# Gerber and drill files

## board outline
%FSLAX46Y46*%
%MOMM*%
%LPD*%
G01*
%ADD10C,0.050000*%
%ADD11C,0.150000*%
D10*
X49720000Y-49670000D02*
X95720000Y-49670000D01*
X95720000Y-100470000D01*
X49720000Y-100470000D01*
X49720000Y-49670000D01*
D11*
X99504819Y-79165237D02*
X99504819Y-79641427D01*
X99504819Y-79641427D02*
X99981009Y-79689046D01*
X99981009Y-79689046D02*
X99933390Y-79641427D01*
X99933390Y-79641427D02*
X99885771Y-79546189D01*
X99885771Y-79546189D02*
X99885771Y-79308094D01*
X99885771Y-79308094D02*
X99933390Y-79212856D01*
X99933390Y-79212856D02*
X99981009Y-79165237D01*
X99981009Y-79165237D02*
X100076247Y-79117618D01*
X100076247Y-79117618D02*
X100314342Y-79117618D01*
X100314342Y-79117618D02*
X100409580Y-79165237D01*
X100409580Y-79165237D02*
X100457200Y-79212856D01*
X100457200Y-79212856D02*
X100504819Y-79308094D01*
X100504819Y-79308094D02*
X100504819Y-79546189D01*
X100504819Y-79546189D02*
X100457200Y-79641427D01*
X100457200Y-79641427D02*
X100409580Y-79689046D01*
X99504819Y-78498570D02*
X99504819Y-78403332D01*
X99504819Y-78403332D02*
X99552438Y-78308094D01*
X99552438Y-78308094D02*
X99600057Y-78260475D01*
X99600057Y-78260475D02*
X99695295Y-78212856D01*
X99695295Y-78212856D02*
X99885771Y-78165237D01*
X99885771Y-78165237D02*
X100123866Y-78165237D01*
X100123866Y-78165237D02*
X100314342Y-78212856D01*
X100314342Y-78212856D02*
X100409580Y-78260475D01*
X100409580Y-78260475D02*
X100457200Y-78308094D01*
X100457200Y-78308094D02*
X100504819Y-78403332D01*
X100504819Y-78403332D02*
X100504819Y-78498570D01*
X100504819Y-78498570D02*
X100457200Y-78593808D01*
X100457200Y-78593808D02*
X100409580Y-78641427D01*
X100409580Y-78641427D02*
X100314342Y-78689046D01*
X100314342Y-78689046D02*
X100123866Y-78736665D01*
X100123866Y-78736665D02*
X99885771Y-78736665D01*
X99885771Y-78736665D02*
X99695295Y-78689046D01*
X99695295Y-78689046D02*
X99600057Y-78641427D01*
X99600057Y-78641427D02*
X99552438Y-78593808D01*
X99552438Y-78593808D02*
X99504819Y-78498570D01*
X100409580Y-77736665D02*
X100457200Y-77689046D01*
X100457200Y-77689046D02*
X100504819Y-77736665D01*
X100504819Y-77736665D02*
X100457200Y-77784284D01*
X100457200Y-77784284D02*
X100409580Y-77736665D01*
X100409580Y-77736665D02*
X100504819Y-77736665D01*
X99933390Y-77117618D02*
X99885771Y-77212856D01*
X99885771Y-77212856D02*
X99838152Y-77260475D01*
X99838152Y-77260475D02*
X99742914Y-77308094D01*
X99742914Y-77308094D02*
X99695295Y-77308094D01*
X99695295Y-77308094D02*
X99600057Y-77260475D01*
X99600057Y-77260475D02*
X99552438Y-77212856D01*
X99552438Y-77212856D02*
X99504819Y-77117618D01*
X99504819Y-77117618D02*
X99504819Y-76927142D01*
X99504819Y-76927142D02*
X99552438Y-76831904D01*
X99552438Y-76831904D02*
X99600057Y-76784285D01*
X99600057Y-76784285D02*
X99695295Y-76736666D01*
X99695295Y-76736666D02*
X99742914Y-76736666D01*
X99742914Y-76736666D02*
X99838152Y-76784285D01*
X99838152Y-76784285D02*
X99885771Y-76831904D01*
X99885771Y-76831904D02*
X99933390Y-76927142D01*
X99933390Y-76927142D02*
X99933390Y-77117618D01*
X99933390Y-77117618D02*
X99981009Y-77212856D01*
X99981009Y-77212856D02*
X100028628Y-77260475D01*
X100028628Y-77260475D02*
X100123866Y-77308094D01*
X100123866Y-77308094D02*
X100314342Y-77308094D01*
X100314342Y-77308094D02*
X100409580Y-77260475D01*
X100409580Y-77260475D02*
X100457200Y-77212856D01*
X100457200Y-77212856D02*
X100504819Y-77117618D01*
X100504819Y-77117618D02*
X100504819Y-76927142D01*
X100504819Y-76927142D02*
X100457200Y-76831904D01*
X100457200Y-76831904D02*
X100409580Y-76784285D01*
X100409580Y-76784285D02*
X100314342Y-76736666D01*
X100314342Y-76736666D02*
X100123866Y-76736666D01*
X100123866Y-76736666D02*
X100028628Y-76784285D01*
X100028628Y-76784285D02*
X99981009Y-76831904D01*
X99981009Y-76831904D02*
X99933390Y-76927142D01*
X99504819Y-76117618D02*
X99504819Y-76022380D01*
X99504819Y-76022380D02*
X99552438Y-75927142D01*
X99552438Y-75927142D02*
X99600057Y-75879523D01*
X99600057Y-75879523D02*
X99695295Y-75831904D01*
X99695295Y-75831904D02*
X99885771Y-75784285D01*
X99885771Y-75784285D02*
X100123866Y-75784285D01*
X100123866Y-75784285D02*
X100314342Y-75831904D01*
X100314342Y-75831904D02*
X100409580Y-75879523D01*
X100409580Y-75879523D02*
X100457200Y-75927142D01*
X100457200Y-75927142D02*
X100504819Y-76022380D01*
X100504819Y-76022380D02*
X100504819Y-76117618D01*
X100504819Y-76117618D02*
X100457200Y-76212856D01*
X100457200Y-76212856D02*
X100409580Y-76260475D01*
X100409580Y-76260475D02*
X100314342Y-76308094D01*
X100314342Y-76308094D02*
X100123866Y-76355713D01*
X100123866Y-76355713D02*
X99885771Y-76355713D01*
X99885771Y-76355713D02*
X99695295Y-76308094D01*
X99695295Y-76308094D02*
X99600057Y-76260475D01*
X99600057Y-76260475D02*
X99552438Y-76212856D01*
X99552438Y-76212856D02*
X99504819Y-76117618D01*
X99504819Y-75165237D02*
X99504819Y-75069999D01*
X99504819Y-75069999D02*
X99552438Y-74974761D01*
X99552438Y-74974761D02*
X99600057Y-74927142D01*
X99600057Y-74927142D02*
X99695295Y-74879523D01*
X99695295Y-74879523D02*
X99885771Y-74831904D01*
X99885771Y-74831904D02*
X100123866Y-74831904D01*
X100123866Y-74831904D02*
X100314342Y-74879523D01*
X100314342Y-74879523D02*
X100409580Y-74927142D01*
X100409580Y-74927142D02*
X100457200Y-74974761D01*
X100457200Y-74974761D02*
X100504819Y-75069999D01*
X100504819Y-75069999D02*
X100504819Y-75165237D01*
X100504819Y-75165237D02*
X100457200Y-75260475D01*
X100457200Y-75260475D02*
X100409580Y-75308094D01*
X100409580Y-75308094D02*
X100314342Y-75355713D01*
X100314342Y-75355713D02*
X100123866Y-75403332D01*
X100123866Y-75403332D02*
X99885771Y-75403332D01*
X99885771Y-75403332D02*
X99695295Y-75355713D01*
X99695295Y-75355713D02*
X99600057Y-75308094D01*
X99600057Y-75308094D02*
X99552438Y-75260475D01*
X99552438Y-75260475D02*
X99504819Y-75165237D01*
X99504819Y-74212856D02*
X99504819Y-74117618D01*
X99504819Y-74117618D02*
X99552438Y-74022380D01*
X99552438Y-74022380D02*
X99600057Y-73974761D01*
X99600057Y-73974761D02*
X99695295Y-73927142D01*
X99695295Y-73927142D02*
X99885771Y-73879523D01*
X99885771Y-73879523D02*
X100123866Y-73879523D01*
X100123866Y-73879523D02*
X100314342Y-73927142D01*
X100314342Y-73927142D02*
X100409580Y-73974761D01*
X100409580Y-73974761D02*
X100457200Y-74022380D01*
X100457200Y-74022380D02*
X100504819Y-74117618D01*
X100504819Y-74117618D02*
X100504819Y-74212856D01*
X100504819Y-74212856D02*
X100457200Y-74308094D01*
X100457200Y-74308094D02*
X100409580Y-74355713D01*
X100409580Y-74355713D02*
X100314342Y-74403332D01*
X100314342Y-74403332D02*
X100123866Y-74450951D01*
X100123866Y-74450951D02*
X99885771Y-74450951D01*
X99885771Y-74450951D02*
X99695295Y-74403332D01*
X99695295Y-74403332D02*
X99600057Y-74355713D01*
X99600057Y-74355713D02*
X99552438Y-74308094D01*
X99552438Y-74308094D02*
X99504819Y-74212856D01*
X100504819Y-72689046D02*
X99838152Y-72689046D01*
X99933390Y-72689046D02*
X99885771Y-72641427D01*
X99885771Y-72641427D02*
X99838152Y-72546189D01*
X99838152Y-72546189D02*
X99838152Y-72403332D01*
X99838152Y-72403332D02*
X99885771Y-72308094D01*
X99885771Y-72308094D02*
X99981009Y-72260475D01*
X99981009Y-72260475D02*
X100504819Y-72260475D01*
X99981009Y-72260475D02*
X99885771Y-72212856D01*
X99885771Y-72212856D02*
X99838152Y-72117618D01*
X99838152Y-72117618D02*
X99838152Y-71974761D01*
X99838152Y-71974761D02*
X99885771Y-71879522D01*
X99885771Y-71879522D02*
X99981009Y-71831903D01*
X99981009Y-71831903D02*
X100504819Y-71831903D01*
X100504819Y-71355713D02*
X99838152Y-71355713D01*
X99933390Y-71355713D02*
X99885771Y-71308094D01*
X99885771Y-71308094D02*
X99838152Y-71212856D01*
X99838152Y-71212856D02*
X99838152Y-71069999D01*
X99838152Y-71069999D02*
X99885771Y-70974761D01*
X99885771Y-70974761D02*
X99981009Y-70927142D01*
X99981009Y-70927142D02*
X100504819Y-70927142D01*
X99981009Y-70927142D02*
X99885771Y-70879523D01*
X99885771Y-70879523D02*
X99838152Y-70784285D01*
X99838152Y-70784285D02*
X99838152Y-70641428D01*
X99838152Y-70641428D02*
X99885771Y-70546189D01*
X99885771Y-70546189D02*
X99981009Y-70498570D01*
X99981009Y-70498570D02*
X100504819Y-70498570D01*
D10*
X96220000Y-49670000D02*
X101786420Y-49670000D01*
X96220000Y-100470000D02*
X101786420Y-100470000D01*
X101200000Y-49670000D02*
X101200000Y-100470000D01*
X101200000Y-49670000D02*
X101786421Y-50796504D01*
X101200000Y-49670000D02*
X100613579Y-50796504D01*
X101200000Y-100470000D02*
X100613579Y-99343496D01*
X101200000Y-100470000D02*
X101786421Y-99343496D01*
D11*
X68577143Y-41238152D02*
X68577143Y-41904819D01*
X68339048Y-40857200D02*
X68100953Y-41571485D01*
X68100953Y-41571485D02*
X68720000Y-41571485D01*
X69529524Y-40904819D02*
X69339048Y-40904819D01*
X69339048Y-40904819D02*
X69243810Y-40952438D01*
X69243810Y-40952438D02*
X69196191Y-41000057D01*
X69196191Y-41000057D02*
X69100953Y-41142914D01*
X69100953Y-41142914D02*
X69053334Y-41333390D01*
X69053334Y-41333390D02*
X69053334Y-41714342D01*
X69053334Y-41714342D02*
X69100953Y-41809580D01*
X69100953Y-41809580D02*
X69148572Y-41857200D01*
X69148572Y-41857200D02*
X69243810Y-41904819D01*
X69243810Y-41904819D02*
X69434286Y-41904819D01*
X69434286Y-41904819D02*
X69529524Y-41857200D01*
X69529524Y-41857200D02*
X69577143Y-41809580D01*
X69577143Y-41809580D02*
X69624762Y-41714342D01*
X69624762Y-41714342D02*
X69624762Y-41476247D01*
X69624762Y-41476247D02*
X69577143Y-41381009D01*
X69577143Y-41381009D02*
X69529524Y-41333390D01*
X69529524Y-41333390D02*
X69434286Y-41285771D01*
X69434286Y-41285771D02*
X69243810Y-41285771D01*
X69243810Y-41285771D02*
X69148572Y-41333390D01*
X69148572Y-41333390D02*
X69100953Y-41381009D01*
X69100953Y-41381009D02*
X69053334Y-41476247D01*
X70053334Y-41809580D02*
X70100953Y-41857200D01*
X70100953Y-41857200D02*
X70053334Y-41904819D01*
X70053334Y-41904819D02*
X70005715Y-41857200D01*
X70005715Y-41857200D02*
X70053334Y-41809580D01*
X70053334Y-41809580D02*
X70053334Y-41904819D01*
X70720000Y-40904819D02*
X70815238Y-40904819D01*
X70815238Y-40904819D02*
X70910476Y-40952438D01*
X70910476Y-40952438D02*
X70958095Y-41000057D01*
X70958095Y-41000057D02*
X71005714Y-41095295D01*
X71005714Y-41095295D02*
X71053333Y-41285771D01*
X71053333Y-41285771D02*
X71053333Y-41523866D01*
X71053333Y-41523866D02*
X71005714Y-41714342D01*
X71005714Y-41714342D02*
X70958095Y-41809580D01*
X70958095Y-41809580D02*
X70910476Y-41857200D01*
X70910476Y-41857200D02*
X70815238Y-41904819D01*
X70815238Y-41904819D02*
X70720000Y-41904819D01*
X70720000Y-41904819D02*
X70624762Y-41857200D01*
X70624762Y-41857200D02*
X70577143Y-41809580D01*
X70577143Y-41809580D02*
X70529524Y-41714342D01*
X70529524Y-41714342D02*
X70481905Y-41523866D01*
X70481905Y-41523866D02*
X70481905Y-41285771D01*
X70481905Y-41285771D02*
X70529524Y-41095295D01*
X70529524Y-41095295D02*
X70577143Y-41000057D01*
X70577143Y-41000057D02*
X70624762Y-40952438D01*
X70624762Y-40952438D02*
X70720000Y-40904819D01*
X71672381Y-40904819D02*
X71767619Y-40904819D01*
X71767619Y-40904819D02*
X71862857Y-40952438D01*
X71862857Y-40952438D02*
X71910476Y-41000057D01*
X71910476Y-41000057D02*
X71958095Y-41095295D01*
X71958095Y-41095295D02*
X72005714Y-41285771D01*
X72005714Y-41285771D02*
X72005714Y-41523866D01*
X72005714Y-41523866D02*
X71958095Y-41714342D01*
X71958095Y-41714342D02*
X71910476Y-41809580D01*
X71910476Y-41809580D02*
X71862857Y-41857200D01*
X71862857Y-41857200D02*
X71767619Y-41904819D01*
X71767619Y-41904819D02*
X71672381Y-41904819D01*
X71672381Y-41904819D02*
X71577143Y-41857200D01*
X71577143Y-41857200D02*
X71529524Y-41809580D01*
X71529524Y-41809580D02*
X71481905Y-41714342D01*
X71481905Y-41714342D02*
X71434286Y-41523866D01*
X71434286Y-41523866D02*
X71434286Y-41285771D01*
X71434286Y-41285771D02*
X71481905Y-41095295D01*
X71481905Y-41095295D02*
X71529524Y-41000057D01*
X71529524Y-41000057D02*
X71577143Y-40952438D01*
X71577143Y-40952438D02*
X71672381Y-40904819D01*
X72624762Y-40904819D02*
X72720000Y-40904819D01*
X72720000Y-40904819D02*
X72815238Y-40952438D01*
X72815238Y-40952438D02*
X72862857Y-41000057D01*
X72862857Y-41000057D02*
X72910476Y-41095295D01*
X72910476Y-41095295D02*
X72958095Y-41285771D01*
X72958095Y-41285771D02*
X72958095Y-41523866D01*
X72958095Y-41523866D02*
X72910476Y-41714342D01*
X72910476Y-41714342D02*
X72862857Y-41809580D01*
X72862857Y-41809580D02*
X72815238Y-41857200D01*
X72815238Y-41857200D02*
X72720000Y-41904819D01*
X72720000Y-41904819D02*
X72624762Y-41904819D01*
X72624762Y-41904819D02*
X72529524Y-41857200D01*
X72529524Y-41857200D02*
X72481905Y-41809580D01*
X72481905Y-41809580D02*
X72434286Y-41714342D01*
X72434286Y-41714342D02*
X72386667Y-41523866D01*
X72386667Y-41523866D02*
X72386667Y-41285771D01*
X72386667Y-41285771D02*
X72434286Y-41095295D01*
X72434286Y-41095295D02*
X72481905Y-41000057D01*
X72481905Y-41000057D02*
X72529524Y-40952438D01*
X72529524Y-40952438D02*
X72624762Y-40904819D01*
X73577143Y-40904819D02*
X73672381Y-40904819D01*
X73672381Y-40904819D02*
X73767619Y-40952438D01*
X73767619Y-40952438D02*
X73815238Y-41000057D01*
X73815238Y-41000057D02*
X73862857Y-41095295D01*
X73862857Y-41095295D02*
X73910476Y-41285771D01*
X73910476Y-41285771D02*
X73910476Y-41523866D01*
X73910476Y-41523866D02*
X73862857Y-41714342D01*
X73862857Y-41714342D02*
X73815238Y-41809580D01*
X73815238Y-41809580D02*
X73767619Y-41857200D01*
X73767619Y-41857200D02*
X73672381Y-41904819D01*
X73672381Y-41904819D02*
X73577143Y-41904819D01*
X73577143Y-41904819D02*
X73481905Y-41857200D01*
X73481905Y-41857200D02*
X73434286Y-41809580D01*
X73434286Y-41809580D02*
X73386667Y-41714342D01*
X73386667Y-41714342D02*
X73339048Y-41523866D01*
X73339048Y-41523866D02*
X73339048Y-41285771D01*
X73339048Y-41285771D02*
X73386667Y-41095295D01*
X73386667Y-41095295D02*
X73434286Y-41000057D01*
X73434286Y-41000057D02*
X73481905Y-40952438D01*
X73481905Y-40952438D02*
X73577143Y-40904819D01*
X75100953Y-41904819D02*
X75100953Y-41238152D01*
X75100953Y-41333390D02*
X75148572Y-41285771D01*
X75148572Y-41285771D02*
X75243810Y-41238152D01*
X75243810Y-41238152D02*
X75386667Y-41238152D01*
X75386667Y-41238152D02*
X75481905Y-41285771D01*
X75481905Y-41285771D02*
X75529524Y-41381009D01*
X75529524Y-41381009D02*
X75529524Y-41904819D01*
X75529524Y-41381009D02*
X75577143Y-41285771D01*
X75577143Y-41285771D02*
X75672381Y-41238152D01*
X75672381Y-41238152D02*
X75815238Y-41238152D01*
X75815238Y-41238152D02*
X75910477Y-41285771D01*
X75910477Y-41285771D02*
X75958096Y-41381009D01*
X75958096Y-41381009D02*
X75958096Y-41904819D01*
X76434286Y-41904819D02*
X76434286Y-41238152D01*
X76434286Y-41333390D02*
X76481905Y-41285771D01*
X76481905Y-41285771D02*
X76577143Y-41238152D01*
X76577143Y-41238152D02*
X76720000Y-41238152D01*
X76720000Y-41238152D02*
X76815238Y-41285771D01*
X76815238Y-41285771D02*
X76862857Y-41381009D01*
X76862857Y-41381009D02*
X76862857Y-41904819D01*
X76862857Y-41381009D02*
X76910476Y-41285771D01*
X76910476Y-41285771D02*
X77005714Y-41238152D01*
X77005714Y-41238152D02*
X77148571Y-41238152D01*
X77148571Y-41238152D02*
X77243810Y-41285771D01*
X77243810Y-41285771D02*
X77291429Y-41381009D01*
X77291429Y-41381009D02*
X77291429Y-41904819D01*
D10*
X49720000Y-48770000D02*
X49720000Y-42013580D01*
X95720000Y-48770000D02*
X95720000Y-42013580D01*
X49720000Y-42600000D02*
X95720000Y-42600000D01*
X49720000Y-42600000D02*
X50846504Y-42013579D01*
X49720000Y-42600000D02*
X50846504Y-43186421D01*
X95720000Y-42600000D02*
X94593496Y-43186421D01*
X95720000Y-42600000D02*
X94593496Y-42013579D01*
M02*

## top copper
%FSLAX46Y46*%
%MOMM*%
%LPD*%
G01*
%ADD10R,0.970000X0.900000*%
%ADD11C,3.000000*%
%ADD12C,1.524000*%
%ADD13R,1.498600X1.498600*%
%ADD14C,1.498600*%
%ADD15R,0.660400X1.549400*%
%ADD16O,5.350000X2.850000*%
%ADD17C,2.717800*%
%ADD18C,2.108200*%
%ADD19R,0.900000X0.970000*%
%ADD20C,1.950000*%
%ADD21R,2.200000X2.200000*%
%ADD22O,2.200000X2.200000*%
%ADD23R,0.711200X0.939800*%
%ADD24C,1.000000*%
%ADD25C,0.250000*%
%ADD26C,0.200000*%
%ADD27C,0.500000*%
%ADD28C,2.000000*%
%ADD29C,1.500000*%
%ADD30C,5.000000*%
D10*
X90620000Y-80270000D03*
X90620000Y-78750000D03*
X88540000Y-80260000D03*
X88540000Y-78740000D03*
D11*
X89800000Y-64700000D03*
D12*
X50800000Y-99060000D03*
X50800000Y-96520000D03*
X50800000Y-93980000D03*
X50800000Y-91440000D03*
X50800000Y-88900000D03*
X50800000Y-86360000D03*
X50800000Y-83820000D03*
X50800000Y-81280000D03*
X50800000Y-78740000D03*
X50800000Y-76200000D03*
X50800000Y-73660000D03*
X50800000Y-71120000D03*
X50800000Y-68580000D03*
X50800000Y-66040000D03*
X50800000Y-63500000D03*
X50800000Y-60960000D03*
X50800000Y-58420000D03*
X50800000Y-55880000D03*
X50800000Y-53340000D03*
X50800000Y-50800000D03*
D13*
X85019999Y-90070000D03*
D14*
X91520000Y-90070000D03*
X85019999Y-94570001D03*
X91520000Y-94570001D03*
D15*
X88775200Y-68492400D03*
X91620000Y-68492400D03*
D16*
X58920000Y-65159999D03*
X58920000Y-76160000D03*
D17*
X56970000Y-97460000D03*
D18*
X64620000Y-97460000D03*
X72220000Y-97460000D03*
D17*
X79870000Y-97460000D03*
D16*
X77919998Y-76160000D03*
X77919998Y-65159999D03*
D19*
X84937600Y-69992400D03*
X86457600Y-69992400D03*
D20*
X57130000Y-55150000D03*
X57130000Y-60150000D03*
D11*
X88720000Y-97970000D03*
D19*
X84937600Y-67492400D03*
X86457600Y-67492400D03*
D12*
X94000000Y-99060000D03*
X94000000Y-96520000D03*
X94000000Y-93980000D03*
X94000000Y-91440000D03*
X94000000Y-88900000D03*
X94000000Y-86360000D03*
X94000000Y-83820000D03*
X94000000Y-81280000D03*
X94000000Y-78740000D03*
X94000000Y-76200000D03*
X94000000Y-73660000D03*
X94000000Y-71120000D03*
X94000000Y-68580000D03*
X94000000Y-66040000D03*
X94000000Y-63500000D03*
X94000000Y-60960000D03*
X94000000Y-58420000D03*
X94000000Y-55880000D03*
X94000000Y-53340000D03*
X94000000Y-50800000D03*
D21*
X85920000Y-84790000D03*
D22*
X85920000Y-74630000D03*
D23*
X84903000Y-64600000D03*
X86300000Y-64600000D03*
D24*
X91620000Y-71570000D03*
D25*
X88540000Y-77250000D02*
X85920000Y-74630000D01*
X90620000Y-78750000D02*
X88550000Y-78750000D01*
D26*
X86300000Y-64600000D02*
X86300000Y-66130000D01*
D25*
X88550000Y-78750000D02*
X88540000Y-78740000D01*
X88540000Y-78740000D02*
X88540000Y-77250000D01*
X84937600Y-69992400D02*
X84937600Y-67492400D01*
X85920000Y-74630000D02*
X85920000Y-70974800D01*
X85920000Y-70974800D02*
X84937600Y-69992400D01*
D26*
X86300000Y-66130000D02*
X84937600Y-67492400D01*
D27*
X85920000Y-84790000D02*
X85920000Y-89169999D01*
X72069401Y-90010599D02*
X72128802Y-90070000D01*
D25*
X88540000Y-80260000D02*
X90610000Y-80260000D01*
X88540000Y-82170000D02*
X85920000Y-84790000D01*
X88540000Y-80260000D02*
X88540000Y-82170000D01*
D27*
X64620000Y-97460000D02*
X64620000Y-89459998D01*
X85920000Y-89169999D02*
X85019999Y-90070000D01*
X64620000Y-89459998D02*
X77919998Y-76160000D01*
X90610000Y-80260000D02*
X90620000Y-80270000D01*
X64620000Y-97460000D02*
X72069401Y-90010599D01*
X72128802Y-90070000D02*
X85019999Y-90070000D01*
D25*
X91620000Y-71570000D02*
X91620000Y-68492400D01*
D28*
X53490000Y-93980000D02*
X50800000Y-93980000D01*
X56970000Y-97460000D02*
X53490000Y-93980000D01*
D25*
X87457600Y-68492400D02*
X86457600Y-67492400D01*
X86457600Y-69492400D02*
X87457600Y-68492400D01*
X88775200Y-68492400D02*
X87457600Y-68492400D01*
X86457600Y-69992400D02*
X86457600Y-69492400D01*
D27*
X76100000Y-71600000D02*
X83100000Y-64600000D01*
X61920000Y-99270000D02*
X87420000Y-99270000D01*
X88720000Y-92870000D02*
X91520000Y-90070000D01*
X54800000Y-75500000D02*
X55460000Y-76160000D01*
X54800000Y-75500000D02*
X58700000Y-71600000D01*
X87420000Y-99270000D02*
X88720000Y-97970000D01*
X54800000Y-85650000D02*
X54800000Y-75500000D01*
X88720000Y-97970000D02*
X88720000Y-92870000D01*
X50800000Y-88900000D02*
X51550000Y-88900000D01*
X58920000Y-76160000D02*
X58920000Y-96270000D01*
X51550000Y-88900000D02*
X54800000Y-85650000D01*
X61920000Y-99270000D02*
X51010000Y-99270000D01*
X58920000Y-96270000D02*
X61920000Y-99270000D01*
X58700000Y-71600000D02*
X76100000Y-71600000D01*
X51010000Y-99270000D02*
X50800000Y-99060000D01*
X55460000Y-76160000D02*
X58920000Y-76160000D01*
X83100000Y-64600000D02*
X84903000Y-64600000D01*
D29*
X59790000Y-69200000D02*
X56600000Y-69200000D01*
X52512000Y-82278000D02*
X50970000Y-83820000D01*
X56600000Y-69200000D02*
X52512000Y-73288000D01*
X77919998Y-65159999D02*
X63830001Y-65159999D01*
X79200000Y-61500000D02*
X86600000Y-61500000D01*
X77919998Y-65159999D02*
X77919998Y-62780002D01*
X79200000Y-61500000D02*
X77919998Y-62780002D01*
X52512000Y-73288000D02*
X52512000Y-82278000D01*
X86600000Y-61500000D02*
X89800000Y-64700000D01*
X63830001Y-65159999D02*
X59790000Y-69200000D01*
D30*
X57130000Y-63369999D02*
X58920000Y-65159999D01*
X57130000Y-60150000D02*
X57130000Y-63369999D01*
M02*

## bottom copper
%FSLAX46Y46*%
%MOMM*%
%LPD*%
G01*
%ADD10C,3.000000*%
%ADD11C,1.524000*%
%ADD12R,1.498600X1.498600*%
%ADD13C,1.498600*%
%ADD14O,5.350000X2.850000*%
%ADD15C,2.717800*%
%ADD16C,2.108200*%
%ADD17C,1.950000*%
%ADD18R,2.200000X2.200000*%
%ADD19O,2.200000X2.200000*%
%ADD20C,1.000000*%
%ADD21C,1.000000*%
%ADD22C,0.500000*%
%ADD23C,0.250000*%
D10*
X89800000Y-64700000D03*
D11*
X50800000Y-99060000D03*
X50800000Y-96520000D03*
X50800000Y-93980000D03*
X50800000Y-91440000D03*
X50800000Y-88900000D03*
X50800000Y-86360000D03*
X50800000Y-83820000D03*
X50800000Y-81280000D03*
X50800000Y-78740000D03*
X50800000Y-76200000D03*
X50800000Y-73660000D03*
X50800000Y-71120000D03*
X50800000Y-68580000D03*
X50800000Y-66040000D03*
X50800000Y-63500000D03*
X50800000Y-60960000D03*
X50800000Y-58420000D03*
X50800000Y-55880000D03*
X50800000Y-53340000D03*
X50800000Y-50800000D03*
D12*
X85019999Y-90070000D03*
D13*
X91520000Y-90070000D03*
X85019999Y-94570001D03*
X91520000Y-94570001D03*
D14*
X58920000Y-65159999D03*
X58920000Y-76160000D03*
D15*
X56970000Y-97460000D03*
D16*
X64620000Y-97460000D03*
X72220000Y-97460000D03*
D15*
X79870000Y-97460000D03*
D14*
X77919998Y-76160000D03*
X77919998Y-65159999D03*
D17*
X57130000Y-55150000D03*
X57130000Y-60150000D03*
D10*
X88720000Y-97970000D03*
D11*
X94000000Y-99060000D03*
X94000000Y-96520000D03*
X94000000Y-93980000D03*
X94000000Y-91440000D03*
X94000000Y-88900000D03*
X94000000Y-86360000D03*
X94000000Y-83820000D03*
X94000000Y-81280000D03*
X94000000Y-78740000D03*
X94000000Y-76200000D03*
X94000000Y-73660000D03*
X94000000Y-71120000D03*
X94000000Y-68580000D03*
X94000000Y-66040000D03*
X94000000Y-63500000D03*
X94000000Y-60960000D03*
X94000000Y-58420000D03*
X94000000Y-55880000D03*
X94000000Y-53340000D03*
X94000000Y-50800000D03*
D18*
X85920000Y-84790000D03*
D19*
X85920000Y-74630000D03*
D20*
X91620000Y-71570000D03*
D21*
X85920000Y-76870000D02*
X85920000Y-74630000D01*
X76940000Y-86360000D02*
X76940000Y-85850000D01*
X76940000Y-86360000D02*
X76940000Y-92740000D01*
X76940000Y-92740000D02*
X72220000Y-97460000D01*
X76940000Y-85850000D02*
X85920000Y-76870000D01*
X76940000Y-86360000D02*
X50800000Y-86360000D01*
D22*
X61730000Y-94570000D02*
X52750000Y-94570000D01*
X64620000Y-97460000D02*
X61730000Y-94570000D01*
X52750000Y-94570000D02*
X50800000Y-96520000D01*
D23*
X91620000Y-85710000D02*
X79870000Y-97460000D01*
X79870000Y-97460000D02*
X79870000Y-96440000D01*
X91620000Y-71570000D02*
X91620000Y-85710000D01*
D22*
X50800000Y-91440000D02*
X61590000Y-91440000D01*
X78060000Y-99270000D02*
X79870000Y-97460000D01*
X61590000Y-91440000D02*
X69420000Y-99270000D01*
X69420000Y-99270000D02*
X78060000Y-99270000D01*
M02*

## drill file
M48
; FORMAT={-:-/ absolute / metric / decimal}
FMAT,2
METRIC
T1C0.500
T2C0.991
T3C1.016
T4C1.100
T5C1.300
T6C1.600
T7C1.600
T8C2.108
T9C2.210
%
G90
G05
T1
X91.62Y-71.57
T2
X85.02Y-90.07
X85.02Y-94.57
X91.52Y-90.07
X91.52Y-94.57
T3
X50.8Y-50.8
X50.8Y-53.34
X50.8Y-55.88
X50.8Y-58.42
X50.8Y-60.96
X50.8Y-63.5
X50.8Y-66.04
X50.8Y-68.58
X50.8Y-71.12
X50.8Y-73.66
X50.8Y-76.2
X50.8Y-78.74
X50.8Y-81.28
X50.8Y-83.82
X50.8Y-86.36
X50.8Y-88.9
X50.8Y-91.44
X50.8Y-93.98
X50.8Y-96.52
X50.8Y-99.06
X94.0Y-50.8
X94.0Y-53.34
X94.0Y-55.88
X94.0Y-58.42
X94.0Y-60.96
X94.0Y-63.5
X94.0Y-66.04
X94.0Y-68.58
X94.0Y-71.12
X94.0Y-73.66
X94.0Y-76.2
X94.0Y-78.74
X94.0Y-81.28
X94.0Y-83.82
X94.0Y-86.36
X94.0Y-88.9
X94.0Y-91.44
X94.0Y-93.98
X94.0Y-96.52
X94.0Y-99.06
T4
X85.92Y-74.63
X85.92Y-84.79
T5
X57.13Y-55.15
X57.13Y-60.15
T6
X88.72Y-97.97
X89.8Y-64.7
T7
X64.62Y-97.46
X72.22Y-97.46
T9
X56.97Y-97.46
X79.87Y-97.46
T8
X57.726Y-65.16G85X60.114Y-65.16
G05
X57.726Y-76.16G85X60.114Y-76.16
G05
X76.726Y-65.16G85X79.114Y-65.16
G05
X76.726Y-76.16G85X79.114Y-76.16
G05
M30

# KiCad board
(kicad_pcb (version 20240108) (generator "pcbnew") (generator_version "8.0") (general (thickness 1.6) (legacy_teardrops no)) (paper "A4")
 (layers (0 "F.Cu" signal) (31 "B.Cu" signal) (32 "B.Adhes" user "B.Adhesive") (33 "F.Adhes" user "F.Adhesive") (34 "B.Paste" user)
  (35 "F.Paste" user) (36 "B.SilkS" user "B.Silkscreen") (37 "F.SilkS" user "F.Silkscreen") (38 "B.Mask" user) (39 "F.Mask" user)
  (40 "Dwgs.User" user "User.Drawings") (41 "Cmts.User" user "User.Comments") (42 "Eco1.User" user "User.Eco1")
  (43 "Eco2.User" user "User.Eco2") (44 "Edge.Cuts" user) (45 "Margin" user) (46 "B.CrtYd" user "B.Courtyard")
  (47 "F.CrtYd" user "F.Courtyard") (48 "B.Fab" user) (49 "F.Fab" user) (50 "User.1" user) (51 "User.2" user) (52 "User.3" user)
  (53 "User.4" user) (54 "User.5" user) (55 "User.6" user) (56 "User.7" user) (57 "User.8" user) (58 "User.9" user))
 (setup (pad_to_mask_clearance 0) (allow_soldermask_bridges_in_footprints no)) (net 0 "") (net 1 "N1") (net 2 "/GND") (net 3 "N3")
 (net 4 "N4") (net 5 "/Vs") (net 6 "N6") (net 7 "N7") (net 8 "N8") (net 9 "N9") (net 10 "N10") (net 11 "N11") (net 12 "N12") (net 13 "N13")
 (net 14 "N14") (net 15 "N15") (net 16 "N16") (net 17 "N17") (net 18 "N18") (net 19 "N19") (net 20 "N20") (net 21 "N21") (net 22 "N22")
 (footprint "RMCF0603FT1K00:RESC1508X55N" (layer "F.Cu") (at 90.62 79.51 90)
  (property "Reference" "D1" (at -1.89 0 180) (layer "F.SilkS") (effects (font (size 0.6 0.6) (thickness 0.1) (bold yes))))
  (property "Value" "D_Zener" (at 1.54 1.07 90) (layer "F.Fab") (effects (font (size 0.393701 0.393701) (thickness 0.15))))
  (pad "1" smd rect (at -0.76 0 90) (size 0.9 0.97) (layers "F.Cu" "F.Paste" "F.Mask") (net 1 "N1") (solder_mask_margin 0.102))
  (pad "2" smd rect (at 0.76 0 90) (size 0.9 0.97) (layers "F.Cu" "F.Paste" "F.Mask") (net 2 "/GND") (solder_mask_margin 0.102)))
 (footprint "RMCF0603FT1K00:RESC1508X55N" (layer "F.Cu") (at 88.54 79.5 90)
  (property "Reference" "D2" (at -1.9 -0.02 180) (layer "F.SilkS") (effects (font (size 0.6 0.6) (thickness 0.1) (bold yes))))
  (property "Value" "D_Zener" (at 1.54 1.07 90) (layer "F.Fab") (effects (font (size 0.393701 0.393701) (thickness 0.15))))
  (pad "1" smd rect (at -0.76 0 90) (size 0.9 0.97) (layers "F.Cu" "F.Paste" "F.Mask") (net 1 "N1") (solder_mask_margin 0.102))
  (pad "2" smd rect (at 0.76 0 90) (size 0.9 0.97) (layers "F.Cu" "F.Paste" "F.Mask") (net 2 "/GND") (solder_mask_margin 0.102)))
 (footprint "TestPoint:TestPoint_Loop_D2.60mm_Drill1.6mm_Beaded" (layer "F.Cu") (at 89.8 64.7)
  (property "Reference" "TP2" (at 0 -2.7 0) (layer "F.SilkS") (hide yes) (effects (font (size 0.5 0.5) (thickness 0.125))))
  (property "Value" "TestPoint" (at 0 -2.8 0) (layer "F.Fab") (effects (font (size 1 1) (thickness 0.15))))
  (pad "1" thru_hole circle (at 0 0) (size 3 3) (drill 1.6) (layers "*.Cu" "*.Mask") (remove_unused_layers no) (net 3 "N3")))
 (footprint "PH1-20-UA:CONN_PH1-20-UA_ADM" (layer "F.Cu") (at 50.8 99.06 90)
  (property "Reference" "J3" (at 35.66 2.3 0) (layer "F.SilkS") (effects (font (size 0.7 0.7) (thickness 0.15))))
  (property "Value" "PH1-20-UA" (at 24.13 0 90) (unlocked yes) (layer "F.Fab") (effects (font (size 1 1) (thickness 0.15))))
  (pad "1" thru_hole circle (at 0 0 90) (size 1.524 1.524) (drill 1.016) (layers "*.Cu" "*.Mask") (remove_unused_layers no) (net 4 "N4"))
  (pad "2" thru_hole circle (at 2.54 0 90) (size 1.524 1.524) (drill 1.016) (layers "*.Cu" "*.Mask") (remove_unused_layers no) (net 1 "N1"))
  (pad "3" thru_hole circle (at 5.08 0 90) (size 1.524 1.524) (drill 1.016) (layers "*.Cu" "*.Mask") (remove_unused_layers no) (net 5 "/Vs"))
  (pad "4" thru_hole circle (at 7.62 0 90) (size 1.524 1.524) (drill 1.016) (layers "*.Cu" "*.Mask") (remove_unused_layers no) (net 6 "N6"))
  (pad "5" thru_hole circle (at 10.16 0 90) (size 1.524 1.524) (drill 1.016) (layers "*.Cu" "*.Mask") (remove_unused_layers no) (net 4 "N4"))
  (pad "6" thru_hole circle (at 12.7 0 90) (size 1.524 1.524) (drill 1.016) (layers "*.Cu" "*.Mask") (remove_unused_layers no)
   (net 2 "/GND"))
  (pad "7" thru_hole circle (at 15.24 0 90) (size 1.524 1.524) (drill 1.016) (layers "*.Cu" "*.Mask") (remove_unused_layers no) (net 3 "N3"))
  (pad "8" thru_hole circle (at 17.78 0 90) (size 1.524 1.524) (drill 1.016) (layers "*.Cu" "*.Mask") (remove_unused_layers no) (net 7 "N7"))
  (pad "9" thru_hole circle (at 20.32 0 90) (size 1.524 1.524) (drill 1.016) (layers "*.Cu" "*.Mask") (remove_unused_layers no) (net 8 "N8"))
  (pad "10" thru_hole circle (at 22.86 0 90) (size 1.524 1.524) (drill 1.016) (layers "*.Cu" "*.Mask") (remove_unused_layers no)
   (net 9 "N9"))
  (pad "11" thru_hole circle (at 25.4 0 90) (size 1.524 1.524) (drill 1.016) (layers "*.Cu" "*.Mask") (remove_unused_layers no)
   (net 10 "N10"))
  (pad "12" thru_hole circle (at 27.94 0 90) (size 1.524 1.524) (drill 1.016) (layers "*.Cu" "*.Mask") (remove_unused_layers no)
   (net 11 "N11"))
  (pad "13" thru_hole circle (at 30.48 0 90) (size 1.524 1.524) (drill 1.016) (layers "*.Cu" "*.Mask") (remove_unused_layers no)
   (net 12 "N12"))
  (pad "14" thru_hole circle (at 33.02 0 90) (size 1.524 1.524) (drill 1.016) (layers "*.Cu" "*.Mask") (remove_unused_layers no)
   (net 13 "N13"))
  (pad "15" thru_hole circle (at 35.56 0 90) (size 1.524 1.524) (drill 1.016) (layers "*.Cu" "*.Mask") (remove_unused_layers no)
   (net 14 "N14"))
  (pad "16" thru_hole circle (at 38.1 0 90) (size 1.524 1.524) (drill 1.016) (layers "*.Cu" "*.Mask") (remove_unused_layers no)
   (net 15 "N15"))
  (pad "17" thru_hole circle (at 40.64 0 90) (size 1.524 1.524) (drill 1.016) (layers "*.Cu" "*.Mask") (remove_unused_layers no)
   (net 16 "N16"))
  (pad "18" thru_hole circle (at 43.18 0 90) (size 1.524 1.524) (drill 1.016) (layers "*.Cu" "*.Mask") (remove_unused_layers no)
   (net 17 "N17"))
  (pad "19" thru_hole circle (at 45.72 0 90) (size 1.524 1.524) (drill 1.016) (layers "*.Cu" "*.Mask") (remove_unused_layers no)
   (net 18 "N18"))
  (pad "20" thru_hole circle (at 48.26 0 90) (size 1.524 1.524) (drill 1.016) (layers "*.Cu" "*.Mask") (remove_unused_layers no)
   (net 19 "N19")))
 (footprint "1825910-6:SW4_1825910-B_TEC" (layer "F.Cu") (at 91.52 94.570001)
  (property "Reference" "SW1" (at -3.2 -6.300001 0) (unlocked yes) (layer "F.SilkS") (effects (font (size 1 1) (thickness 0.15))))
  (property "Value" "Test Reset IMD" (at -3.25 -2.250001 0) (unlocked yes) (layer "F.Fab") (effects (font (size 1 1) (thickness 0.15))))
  (pad "1" thru_hole rect (at -6.500001 -4.500001) (size 1.4986 1.4986) (drill 0.9906) (layers "*.Cu" "*.Mask") (remove_unused_layers no)
   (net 1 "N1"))
  (pad "2" thru_hole circle (at 0 -4.500001) (size 1.4986 1.4986) (drill 0.9906) (layers "*.Cu" "*.Mask") (remove_unused_layers no)
   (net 4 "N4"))
  (pad "3" thru_hole circle (at -6.500001 0) (size 1.4986 1.4986) (drill 0.9906) (layers "*.Cu" "*.Mask") (remove_unused_layers no))
  (pad "4" thru_hole circle (at 0 0) (size 1.4986 1.4986) (drill 0.9906) (layers "*.Cu" "*.Mask") (remove_unused_layers no)))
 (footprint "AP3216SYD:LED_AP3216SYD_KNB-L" (layer "F.Cu") (at 90.1976 68.4924)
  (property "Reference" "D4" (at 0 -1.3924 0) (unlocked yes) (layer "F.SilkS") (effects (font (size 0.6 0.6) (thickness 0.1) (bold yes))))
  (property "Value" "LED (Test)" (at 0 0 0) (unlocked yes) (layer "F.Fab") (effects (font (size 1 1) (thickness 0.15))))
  (pad "1" smd rect (at -1.4224 0) (size 0.6604 1.5494) (layers "F.Cu" "F.Paste" "F.Mask") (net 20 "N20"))
  (pad "2" smd rect (at 1.4224 0) (size 0.6604 1.5494) (layers "F.Cu" "F.Paste" "F.Mask") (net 6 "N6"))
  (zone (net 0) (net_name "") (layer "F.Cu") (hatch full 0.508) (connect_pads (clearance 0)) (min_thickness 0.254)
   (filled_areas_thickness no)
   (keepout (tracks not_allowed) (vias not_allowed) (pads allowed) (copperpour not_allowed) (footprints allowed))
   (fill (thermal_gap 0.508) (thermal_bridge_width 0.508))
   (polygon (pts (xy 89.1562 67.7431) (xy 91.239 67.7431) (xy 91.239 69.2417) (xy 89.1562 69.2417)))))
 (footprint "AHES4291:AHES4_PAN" (layer "F.Cu") (at 58.919999 65.159998)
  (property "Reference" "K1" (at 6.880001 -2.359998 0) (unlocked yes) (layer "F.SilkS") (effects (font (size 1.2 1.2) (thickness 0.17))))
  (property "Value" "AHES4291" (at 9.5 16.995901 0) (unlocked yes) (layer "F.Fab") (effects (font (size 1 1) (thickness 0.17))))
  (pad "1" thru_hole oval (at 0.000001 0.000001) (size 5.35 2.85) (drill oval 4.4958 2.1082) (layers "*.Cu" "*.Mask")
   (remove_unused_layers no) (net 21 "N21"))
  (pad "2" thru_hole oval (at 0.000001 11.000002) (size 5.35 2.85) (drill oval 4.4958 2.1082) (layers "*.Cu" "*.Mask")
   (remove_unused_layers no) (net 4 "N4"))
  (pad "3" thru_hole circle (at -1.949999 32.300002) (size 2.7178 2.7178) (drill 2.2098) (layers "*.Cu" "*.Mask") (remove_unused_layers no)
   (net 5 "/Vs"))
  (pad "4" thru_hole circle (at 5.700001 32.300002) (size 2.1082 2.1082) (drill 1.6002) (layers "*.Cu" "*.Mask") (remove_unused_layers no)
   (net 1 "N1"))
  (pad "5" thru_hole circle (at 13.300001 32.300002) (size 2.1082 2.1082) (drill 1.6002) (layers "*.Cu" "*.Mask") (remove_unused_layers no)
   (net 2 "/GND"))
  (pad "6" thru_hole circle (at 20.950001 32.300002) (size 2.7178 2.7178) (drill 2.2098) (layers "*.Cu" "*.Mask") (remove_unused_layers no)
   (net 6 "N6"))
  (pad "7" thru_hole oval (at 18.999999 11.000002) (size 5.35 2.85) (drill oval 4.4958 2.1082) (layers "*.Cu" "*.Mask")
   (remove_unused_layers no) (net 1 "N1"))
  (pad "8" thru_hole oval (at 18.999999 0.000001) (size 5.35 2.85) (drill oval 4.4958 2.1082) (layers "*.Cu" "*.Mask")
   (remove_unused_layers no) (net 3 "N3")))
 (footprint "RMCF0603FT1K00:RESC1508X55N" (layer "F.Cu") (at 85.6976 69.9924)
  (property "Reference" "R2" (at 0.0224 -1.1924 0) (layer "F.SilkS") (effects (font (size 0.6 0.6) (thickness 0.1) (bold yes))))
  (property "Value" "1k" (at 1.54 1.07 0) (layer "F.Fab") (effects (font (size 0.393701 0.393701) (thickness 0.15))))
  (pad "1" smd rect (at -0.76 0) (size 0.9 0.97) (layers "F.Cu" "F.Paste" "F.Mask") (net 2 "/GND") (solder_mask_margin 0.102))
  (pad "2" smd rect (at 0.76 0) (size 0.9 0.97) (layers "F.Cu" "F.Paste" "F.Mask") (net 20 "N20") (solder_mask_margin 0.102)))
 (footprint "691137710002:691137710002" (layer "F.Cu") (at 57.13 57.65 -90)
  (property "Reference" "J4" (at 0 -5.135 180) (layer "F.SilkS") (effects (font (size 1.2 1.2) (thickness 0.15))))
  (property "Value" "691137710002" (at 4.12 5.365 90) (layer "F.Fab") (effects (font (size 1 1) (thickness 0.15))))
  (pad "1" thru_hole circle (at -2.5 0 270) (size 1.95 1.95) (drill 1.3) (layers "*.Cu" "*.Mask") (remove_unused_layers no) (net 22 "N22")
   (solder_mask_margin 0.102))
  (pad "2" thru_hole circle (at 2.5 0 270) (size 1.95 1.95) (drill 1.3) (layers "*.Cu" "*.Mask") (remove_unused_layers no) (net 21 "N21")
   (solder_mask_margin 0.102)))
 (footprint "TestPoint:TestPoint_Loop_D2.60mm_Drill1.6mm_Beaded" (layer "F.Cu") (at 88.72 97.97)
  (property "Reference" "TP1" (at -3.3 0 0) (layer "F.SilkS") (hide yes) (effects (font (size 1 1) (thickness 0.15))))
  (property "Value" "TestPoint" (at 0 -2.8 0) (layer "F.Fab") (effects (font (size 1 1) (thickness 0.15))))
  (pad "1" thru_hole circle (at 0 0) (size 3 3) (drill 1.6) (layers "*.Cu" "*.Mask") (remove_unused_layers no) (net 4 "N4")))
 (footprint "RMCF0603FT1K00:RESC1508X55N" (layer "F.Cu") (at 85.6976 67.4924)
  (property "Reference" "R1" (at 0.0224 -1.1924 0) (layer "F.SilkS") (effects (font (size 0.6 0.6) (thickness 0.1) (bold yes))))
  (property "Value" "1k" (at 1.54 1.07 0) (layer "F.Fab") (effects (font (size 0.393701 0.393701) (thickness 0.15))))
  (pad "1" smd rect (at -0.76 0) (size 0.9 0.97) (layers "F.Cu" "F.Paste" "F.Mask") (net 2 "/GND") (solder_mask_margin 0.102))
  (pad "2" smd rect (at 0.76 0) (size 0.9 0.97) (layers "F.Cu" "F.Paste" "F.Mask") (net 20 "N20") (solder_mask_margin 0.102)))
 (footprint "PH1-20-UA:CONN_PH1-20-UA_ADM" (layer "F.Cu") (at 94 99.06 90)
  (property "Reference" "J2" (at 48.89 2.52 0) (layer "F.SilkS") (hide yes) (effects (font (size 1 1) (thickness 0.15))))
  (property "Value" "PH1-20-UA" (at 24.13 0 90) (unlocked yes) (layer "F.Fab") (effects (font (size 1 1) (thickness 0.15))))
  (pad "1" thru_hole circle (at 0 0 90) (size 1.524 1.524) (drill 1.016) (layers "*.Cu" "*.Mask") (remove_unused_layers no))
  (pad "2" thru_hole circle (at 2.54 0 90) (size 1.524 1.524) (drill 1.016) (layers "*.Cu" "*.Mask") (remove_unused_layers no))
  (pad "3" thru_hole circle (at 5.08 0 90) (size 1.524 1.524) (drill 1.016) (layers "*.Cu" "*.Mask") (remove_unused_layers no))
  (pad "4" thru_hole circle (at 7.62 0 90) (size 1.524 1.524) (drill 1.016) (layers "*.Cu" "*.Mask") (remove_unused_layers no))
  (pad "5" thru_hole circle (at 10.16 0 90) (size 1.524 1.524) (drill 1.016) (layers "*.Cu" "*.Mask") (remove_unused_layers no))
  (pad "6" thru_hole circle (at 12.7 0 90) (size 1.524 1.524) (drill 1.016) (layers "*.Cu" "*.Mask") (remove_unused_layers no))
  (pad "7" thru_hole circle (at 15.24 0 90) (size 1.524 1.524) (drill 1.016) (layers "*.Cu" "*.Mask") (remove_unused_layers no))
  (pad "8" thru_hole circle (at 17.78 0 90) (size 1.524 1.524) (drill 1.016) (layers "*.Cu" "*.Mask") (remove_unused_layers no))
  (pad "9" thru_hole circle (at 20.32 0 90) (size 1.524 1.524) (drill 1.016) (layers "*.Cu" "*.Mask") (remove_unused_layers no))
  (pad "10" thru_hole circle (at 22.86 0 90) (size 1.524 1.524) (drill 1.016) (layers "*.Cu" "*.Mask") (remove_unused_layers no))
  (pad "11" thru_hole circle (at 25.4 0 90) (size 1.524 1.524) (drill 1.016) (layers "*.Cu" "*.Mask") (remove_unused_layers no))
  (pad "12" thru_hole circle (at 27.94 0 90) (size 1.524 1.524) (drill 1.016) (layers "*.Cu" "*.Mask") (remove_unused_layers no))
  (pad "13" thru_hole circle (at 30.48 0 90) (size 1.524 1.524) (drill 1.016) (layers "*.Cu" "*.Mask") (remove_unused_layers no))
  (pad "14" thru_hole circle (at 33.02 0 90) (size 1.524 1.524) (drill 1.016) (layers "*.Cu" "*.Mask") (remove_unused_layers no))
  (pad "15" thru_hole circle (at 35.56 0 90) (size 1.524 1.524) (drill 1.016) (layers "*.Cu" "*.Mask") (remove_unused_layers no))
  (pad "16" thru_hole circle (at 38.1 0 90) (size 1.524 1.524) (drill 1.016) (layers "*.Cu" "*.Mask") (remove_unused_layers no))
  (pad "17" thru_hole circle (at 40.64 0 90) (size 1.524 1.524) (drill 1.016) (layers "*.Cu" "*.Mask") (remove_unused_layers no))
  (pad "18" thru_hole circle (at 43.18 0 90) (size 1.524 1.524) (drill 1.016) (layers "*.Cu" "*.Mask") (remove_unused_layers no))
  (pad "19" thru_hole circle (at 45.72 0 90) (size 1.524 1.524) (drill 1.016) (layers "*.Cu" "*.Mask") (remove_unused_layers no))
  (pad "20" thru_hole circle (at 48.26 0 90) (size 1.524 1.524) (drill 1.016) (layers "*.Cu" "*.Mask") (remove_unused_layers no)))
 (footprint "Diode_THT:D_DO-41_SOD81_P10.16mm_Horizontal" (layer "F.Cu") (at 85.92 84.79 90)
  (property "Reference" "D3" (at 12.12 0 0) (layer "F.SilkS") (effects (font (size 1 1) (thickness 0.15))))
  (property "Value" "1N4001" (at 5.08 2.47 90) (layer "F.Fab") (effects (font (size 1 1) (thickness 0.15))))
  (pad "1" thru_hole rect (at 0 0 90) (size 2.2 2.2) (drill 1.1) (layers "*.Cu" "*.Mask") (remove_unused_layers no) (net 1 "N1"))
  (pad "2" thru_hole oval (at 10.16 0 90) (size 2.2 2.2) (drill 1.1) (layers "*.Cu" "*.Mask") (remove_unused_layers no) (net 2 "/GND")))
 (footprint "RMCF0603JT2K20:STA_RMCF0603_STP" (layer "F.Cu") (at 85.6015 64.6)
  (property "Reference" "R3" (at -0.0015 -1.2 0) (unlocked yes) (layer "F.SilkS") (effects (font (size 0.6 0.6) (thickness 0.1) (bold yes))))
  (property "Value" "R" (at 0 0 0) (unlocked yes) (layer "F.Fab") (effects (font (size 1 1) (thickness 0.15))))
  (pad "1" smd rect (at -0.6985 0) (size 0.7112 0.9398) (layers "F.Cu" "F.Paste" "F.Mask") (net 4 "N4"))
  (pad "2" smd rect (at 0.6985 0) (size 0.7112 0.9398) (layers "F.Cu" "F.Paste" "F.Mask") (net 2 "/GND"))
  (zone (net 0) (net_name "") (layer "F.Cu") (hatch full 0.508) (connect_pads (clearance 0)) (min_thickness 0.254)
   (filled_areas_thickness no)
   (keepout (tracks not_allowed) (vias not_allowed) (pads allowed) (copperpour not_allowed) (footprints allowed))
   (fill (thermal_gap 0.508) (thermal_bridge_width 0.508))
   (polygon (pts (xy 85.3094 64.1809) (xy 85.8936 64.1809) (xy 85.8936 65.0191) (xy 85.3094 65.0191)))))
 (gr_rect (start 49.72 49.67) (end 95.72 100.47) (stroke (width 0.05) (type default)) (fill none) (layer "Edge.Cuts"))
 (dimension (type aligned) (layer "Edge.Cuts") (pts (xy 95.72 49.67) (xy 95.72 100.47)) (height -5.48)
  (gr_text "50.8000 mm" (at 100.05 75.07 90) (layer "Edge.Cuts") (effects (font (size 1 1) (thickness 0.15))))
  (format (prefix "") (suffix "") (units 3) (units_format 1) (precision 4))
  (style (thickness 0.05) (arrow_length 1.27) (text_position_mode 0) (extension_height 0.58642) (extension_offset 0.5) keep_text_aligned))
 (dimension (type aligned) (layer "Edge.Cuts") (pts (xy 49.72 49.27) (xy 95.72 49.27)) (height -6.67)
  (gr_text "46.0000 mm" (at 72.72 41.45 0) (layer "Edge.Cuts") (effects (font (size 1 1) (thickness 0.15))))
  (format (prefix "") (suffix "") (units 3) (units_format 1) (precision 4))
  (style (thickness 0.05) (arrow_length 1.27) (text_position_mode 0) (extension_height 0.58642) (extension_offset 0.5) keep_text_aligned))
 (segment (start 88.54 77.25) (end 85.92 74.63) (width 0.25) (layer "F.Cu") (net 2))
 (segment (start 90.62 78.75) (end 88.55 78.75) (width 0.25) (layer "F.Cu") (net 2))
 (segment (start 86.3 64.6) (end 86.3 66.13) (width 0.2) (layer "F.Cu") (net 2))
 (segment (start 88.55 78.75) (end 88.54 78.74) (width 0.25) (layer "F.Cu") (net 2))
 (segment (start 88.54 78.74) (end 88.54 77.25) (width 0.25) (layer "F.Cu") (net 2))
 (segment (start 84.9376 69.9924) (end 84.9376 67.4924) (width 0.25) (layer "F.Cu") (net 2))
 (segment (start 85.92 74.63) (end 85.92 70.9748) (width 0.25) (layer "F.Cu") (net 2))
 (segment (start 85.92 70.9748) (end 84.9376 69.9924) (width 0.25) (layer "F.Cu") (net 2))
 (segment (start 86.3 66.13) (end 84.9376 67.4924) (width 0.2) (layer "F.Cu") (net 2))
 (segment (start 85.92 76.87) (end 85.92 74.63) (width 1) (layer "B.Cu") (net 2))
 (segment (start 76.94 86.36) (end 76.94 85.85) (width 1) (layer "B.Cu") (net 2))
 (segment (start 76.94 86.36) (end 76.94 92.74) (width 1) (layer "B.Cu") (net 2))
 (segment (start 76.94 92.74) (end 72.22 97.46) (width 1) (layer "B.Cu") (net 2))
 (segment (start 76.94 85.85) (end 85.92 76.87) (width 1) (layer "B.Cu") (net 2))
 (segment (start 76.94 86.36) (end 50.8 86.36) (width 1) (layer "B.Cu") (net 2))
 (segment (start 85.92 84.79) (end 85.92 89.169999) (width 0.5) (layer "F.Cu") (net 1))
 (segment (start 72.069401 90.010599) (end 72.128802 90.07) (width 0.5) (layer "F.Cu") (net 1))
 (segment (start 88.54 80.26) (end 90.61 80.26) (width 0.25) (layer "F.Cu") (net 1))
 (segment (start 88.54 82.17) (end 85.92 84.79) (width 0.25) (layer "F.Cu") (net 1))
 (segment (start 88.54 80.26) (end 88.54 82.17) (width 0.25) (layer "F.Cu") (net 1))
 (segment (start 64.62 97.46) (end 64.62 89.459998) (width 0.5) (layer "F.Cu") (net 1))
 (segment (start 85.92 89.169999) (end 85.019999 90.07) (width 0.5) (layer "F.Cu") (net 1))
 (segment (start 64.62 89.459998) (end 77.919998 76.16) (width 0.5) (layer "F.Cu") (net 1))
 (segment (start 90.61 80.26) (end 90.62 80.27) (width 0.5) (layer "F.Cu") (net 1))
 (segment (start 64.62 97.46) (end 72.069401 90.010599) (width 0.5) (layer "F.Cu") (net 1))
 (segment (start 72.128802 90.07) (end 85.019999 90.07) (width 0.5) (layer "F.Cu") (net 1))
 (segment (start 61.73 94.57) (end 52.75 94.57) (width 0.5) (layer "B.Cu") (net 1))
 (segment (start 64.62 97.46) (end 61.73 94.57) (width 0.5) (layer "B.Cu") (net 1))
 (segment (start 52.75 94.57) (end 50.8 96.52) (width 0.5) (layer "B.Cu") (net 1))
 (segment (start 91.62 71.57) (end 91.62 68.4924) (width 0.25) (layer "F.Cu") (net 6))
 (via (at 91.62 71.57) (size 1) (drill 0.5) (layers "F.Cu" "B.Cu") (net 6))
 (segment (start 91.62 85.71) (end 79.87 97.46) (width 0.25) (layer "B.Cu") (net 6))
 (segment (start 79.87 97.46) (end 79.87 96.44) (width 0.25) (layer "B.Cu") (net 6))
 (segment (start 91.62 71.57) (end 91.62 85.71) (width 0.25) (layer "B.Cu") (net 6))
 (segment (start 50.8 91.44) (end 61.59 91.44) (width 0.5) (layer "B.Cu") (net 6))
 (segment (start 78.06 99.27) (end 79.87 97.46) (width 0.5) (layer "B.Cu") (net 6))
 (segment (start 61.59 91.44) (end 69.42 99.27) (width 0.5) (layer "B.Cu") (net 6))
 (segment (start 69.42 99.27) (end 78.06 99.27) (width 0.5) (layer "B.Cu") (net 6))
 (segment (start 53.49 93.98) (end 50.8 93.98) (width 2) (layer "F.Cu") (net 5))
 (segment (start 56.97 97.46) (end 53.49 93.98) (width 2) (layer "F.Cu") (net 5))
 (segment (start 87.4576 68.4924) (end 86.4576 67.4924) (width 0.25) (layer "F.Cu") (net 20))
 (segment (start 86.4576 69.4924) (end 87.4576 68.4924) (width 0.25) (layer "F.Cu") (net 20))
 (segment (start 88.7752 68.4924) (end 87.4576 68.4924) (width 0.25) (layer "F.Cu") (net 20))
 (segment (start 86.4576 69.9924) (end 86.4576 69.4924) (width 0.25) (layer "F.Cu") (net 20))
 (segment (start 76.1 71.6) (end 83.1 64.6) (width 0.5) (layer "F.Cu") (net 4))
 (segment (start 61.92 99.27) (end 87.42 99.27) (width 0.5) (layer "F.Cu") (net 4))
 (segment (start 88.72 92.87) (end 91.52 90.07) (width 0.5) (layer "F.Cu") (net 4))
 (segment (start 54.8 75.5) (end 55.46 76.16) (width 0.5) (layer "F.Cu") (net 4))
 (segment (start 54.8 75.5) (end 58.7 71.6) (width 0.5) (layer "F.Cu") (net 4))
 (segment (start 87.42 99.27) (end 88.72 97.97) (width 0.5) (layer "F.Cu") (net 4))
 (segment (start 54.8 85.65) (end 54.8 75.5) (width 0.5) (layer "F.Cu") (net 4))
 (segment (start 88.72 97.97) (end 88.72 92.87) (width 0.5) (layer "F.Cu") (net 4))
 (segment (start 50.8 88.9) (end 51.55 88.9) (width 0.5) (layer "F.Cu") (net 4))
 (segment (start 58.92 76.16) (end 58.92 96.27) (width 0.5) (layer "F.Cu") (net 4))
 (segment (start 51.55 88.9) (end 54.8 85.65) (width 0.5) (layer "F.Cu") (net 4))
 (segment (start 61.92 99.27) (end 51.01 99.27) (width 0.5) (layer "F.Cu") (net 4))
 (segment (start 58.92 96.27) (end 61.92 99.27) (width 0.5) (layer "F.Cu") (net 4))
 (segment (start 58.7 71.6) (end 76.1 71.6) (width 0.5) (layer "F.Cu") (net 4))
 (segment (start 51.01 99.27) (end 50.8 99.06) (width 0.5) (layer "F.Cu") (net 4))
 (segment (start 55.46 76.16) (end 58.92 76.16) (width 0.5) (layer "F.Cu") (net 4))
 (segment (start 83.1 64.6) (end 84.903 64.6) (width 0.5) (layer "F.Cu") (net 4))
 (segment (start 59.79 69.2) (end 56.6 69.2) (width 1.5) (layer "F.Cu") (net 3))
 (segment (start 52.512 82.278) (end 50.97 83.82) (width 1.5) (layer "F.Cu") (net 3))
 (segment (start 56.6 69.2) (end 52.512 73.288) (width 1.5) (layer "F.Cu") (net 3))
 (segment (start 77.919998 65.159999) (end 63.830001 65.159999) (width 1.5) (layer "F.Cu") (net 3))
 (segment (start 79.2 61.5) (end 86.6 61.5) (width 1.5) (layer "F.Cu") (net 3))
 (segment (start 77.919998 65.159999) (end 77.919998 62.780002) (width 1.5) (layer "F.Cu") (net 3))
 (segment (start 79.2 61.5) (end 77.919998 62.780002) (width 1.5) (layer "F.Cu") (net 3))
 (segment (start 52.512 73.288) (end 52.512 82.278) (width 1.5) (layer "F.Cu") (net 3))
 (segment (start 86.6 61.5) (end 89.8 64.7) (width 1.5) (layer "F.Cu") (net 3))
 (segment (start 63.830001 65.159999) (end 59.79 69.2) (width 1.5) (layer "F.Cu") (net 3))
 (segment (start 57.13 63.369999) (end 58.92 65.159999) (width 5) (layer "F.Cu") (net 21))
 (segment (start 57.13 60.15) (end 57.13 63.369999) (width 5) (layer "F.Cu") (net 21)))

